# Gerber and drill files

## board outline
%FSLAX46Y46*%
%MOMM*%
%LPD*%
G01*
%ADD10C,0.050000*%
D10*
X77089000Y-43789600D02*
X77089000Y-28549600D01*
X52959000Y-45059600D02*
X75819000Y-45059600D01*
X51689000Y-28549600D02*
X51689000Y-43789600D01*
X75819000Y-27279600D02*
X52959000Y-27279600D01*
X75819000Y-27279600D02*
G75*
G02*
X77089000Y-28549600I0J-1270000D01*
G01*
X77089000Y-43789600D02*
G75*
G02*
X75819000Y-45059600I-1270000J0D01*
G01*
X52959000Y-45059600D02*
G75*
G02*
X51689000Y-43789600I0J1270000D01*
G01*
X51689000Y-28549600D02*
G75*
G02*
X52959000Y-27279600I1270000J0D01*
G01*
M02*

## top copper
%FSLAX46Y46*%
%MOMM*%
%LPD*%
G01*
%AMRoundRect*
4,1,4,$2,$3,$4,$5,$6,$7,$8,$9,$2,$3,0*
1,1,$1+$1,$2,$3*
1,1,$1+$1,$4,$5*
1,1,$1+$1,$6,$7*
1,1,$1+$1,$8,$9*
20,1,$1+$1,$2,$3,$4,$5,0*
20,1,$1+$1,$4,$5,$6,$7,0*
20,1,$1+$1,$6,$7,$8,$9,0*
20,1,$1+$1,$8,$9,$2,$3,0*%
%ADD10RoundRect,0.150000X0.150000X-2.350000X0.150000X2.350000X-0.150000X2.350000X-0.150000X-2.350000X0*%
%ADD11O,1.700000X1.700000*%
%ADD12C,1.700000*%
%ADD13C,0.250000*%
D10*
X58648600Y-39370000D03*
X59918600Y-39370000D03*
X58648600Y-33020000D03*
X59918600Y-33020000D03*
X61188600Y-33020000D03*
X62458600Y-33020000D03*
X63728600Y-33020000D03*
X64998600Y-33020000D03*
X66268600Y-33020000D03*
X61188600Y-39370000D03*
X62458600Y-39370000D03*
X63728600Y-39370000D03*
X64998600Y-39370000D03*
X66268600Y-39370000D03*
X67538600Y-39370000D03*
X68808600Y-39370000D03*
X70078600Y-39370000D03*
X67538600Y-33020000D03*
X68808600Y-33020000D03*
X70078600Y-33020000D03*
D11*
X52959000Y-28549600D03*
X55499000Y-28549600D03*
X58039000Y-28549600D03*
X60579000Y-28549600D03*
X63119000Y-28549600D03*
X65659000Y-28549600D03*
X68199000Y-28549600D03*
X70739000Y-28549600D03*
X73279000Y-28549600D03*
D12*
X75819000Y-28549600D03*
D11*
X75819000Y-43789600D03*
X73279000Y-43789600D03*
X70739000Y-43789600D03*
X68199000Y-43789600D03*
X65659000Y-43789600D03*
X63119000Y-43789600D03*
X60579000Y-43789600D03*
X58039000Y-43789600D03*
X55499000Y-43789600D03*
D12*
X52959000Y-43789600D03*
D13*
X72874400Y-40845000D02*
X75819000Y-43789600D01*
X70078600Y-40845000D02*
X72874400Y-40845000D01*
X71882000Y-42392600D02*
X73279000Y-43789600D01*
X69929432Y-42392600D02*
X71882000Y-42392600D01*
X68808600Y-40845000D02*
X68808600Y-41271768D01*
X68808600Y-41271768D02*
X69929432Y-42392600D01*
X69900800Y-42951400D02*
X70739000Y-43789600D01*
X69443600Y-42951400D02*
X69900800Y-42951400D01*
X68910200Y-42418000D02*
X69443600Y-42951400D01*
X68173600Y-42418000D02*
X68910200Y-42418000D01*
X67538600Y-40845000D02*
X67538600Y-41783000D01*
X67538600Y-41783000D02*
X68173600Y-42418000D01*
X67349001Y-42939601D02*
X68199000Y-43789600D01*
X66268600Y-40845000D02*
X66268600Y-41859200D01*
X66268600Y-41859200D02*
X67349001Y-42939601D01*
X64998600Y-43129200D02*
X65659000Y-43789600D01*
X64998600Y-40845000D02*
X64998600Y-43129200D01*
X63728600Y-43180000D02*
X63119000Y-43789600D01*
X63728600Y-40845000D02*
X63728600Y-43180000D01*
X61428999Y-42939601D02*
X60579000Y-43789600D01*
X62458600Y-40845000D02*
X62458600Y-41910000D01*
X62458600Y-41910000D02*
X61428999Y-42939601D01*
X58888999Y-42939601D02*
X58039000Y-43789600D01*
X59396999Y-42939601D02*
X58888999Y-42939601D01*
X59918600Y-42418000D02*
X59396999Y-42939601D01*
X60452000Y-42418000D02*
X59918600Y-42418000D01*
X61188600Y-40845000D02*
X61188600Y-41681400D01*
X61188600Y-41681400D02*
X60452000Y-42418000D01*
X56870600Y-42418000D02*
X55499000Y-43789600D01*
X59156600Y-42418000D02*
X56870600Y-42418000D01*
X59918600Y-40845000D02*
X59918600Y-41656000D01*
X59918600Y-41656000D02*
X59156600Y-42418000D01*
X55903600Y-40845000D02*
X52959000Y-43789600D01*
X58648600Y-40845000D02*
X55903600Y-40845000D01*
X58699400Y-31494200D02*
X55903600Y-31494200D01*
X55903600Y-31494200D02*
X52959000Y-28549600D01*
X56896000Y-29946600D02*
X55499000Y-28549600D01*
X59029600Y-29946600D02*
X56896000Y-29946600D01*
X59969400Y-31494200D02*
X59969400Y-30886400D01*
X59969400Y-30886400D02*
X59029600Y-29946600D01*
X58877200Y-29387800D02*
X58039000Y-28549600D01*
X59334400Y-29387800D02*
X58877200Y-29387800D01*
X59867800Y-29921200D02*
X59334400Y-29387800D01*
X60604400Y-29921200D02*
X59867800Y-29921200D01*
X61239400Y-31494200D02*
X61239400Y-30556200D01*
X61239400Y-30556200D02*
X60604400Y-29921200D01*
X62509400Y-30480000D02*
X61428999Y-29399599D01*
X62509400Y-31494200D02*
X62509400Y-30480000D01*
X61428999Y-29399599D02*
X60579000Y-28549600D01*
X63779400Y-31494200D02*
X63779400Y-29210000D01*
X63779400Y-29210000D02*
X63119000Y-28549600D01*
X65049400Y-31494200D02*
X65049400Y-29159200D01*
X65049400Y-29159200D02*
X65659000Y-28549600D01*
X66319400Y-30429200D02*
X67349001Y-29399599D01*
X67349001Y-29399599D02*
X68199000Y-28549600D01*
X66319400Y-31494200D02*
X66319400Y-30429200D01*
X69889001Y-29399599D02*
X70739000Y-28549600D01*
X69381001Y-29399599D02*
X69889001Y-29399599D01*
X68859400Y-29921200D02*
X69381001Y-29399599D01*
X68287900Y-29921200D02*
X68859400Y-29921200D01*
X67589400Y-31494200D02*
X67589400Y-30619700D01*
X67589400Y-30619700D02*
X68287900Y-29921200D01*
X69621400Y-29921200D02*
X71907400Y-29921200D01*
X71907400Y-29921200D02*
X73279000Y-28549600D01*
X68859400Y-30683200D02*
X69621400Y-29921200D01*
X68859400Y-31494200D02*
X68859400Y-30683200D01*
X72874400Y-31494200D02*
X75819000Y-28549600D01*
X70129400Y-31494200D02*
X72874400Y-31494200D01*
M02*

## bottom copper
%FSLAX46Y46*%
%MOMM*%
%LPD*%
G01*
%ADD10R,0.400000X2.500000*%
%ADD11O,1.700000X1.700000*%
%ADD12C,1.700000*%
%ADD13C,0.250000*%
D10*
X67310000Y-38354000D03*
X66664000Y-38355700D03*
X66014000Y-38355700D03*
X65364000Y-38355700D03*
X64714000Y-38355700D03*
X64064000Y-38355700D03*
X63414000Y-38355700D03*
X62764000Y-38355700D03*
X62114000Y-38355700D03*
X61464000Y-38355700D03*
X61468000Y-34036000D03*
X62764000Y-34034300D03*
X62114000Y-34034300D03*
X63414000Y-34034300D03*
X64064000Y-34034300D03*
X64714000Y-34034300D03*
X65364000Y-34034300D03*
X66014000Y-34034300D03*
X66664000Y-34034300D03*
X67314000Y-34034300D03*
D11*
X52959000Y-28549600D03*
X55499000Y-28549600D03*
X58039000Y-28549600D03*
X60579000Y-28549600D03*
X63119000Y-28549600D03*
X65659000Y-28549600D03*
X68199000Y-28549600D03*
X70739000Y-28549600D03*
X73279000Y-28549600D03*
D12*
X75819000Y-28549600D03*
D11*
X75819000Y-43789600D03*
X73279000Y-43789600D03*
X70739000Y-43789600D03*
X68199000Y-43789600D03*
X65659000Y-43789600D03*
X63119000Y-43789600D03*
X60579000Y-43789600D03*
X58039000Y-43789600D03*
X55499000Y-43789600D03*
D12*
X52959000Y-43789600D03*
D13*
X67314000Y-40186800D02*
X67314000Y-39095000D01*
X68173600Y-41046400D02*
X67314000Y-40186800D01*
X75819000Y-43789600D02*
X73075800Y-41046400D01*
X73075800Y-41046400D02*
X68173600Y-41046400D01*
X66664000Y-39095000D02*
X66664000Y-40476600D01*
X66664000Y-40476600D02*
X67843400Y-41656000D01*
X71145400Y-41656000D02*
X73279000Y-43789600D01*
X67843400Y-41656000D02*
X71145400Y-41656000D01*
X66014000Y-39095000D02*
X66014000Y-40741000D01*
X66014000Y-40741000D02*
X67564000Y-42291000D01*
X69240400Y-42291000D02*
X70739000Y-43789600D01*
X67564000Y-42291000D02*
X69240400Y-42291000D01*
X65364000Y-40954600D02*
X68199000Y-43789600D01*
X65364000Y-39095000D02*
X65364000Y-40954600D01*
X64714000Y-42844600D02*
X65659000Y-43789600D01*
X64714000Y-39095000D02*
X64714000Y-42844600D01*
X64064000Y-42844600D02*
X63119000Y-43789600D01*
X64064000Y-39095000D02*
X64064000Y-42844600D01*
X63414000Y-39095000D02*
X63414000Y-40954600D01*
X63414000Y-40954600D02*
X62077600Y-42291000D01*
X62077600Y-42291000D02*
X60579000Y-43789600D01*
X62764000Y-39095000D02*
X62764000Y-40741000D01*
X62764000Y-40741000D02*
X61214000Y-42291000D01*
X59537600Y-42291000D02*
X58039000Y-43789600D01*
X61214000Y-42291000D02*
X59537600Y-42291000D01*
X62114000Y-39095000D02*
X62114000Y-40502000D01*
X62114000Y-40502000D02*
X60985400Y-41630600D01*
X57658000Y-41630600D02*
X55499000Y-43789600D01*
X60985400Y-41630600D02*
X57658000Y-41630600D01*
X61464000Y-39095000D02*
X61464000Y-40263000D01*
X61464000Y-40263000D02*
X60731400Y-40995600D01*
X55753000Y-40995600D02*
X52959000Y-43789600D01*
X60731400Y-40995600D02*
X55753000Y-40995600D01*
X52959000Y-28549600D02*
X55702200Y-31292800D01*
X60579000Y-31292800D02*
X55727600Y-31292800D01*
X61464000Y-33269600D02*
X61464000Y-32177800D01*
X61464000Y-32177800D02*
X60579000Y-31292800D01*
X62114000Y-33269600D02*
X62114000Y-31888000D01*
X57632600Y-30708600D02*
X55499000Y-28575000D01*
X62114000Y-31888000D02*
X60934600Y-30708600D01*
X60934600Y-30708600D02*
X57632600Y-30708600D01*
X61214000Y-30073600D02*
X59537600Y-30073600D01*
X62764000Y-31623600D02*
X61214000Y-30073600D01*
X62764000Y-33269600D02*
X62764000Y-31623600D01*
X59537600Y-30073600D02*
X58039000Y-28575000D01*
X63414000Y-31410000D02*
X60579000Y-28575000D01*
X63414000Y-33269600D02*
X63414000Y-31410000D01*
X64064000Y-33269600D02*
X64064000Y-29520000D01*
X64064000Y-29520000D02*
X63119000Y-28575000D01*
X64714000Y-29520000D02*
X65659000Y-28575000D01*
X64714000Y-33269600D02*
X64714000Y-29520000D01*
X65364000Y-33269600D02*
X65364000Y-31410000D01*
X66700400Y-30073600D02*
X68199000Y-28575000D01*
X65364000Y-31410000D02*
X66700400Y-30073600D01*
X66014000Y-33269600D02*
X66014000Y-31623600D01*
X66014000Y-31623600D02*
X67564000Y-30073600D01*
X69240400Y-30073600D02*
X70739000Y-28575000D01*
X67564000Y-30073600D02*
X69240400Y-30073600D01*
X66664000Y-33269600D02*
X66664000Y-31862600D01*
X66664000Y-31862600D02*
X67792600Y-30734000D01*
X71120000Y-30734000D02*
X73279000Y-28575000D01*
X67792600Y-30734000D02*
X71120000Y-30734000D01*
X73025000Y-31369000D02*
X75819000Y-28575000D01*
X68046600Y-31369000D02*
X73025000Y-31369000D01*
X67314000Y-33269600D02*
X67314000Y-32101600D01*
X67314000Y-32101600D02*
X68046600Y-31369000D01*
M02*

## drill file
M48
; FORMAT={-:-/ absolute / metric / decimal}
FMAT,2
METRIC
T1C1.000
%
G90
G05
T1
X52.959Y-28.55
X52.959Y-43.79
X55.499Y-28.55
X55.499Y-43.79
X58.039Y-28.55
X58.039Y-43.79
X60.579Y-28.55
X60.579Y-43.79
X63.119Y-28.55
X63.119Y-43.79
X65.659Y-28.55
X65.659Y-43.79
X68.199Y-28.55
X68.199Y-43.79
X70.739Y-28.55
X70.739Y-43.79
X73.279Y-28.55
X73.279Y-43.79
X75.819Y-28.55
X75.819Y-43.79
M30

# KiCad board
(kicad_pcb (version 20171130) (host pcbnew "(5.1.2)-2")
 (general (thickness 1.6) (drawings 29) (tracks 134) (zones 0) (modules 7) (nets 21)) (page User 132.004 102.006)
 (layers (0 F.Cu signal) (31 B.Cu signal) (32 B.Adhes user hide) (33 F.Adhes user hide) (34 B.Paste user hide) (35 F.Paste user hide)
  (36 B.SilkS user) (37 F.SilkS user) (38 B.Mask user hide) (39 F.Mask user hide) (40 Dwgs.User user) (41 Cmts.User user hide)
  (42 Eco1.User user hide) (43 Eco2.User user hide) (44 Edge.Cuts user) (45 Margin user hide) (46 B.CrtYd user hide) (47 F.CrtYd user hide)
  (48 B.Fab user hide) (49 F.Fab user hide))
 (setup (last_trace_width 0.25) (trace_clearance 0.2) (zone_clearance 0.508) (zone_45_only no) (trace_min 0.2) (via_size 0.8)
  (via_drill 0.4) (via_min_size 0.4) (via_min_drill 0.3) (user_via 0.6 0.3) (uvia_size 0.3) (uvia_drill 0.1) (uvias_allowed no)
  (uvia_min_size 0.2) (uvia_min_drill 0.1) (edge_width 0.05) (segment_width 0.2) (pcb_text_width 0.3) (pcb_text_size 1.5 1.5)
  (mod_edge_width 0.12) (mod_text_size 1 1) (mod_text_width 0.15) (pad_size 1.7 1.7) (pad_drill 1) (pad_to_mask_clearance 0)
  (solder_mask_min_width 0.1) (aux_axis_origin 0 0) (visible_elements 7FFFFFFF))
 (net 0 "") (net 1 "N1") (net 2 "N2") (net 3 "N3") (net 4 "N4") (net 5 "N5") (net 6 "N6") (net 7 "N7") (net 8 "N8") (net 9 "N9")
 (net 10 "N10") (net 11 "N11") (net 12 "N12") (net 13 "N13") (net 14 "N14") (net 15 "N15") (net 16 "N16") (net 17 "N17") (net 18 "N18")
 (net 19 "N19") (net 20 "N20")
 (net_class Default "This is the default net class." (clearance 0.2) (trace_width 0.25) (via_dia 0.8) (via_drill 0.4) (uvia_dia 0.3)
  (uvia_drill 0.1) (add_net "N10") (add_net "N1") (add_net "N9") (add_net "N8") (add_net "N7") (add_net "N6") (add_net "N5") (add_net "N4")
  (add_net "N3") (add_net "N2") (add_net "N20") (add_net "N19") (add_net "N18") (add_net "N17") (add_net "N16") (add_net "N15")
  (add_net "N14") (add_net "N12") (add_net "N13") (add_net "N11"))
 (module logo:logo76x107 (layer B.Cu) (at 72.4535 36.322 90)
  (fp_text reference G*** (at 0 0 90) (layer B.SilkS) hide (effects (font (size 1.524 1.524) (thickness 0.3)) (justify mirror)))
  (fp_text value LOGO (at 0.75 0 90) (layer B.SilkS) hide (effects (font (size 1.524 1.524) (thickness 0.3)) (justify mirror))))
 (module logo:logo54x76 (layer F.Cu) (at 54.864 36.195 90)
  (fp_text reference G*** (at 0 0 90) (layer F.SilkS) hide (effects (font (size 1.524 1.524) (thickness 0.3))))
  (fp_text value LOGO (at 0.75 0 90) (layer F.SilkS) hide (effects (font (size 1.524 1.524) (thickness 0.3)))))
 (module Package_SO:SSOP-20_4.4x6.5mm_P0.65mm (layer B.Cu) (at 64.389 36.195 90)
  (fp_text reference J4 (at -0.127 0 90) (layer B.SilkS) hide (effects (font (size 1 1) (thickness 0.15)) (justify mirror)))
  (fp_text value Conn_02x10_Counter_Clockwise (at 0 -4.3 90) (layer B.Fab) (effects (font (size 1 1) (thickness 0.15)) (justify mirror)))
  (pad 1 smd rect (at -2.159 2.921 90) (size 2.5 0.4) (layers B.Cu B.Paste B.Mask) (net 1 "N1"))
  (pad 2 smd rect (at -2.1607 2.275 90) (size 2.5 0.4) (layers B.Cu B.Paste B.Mask) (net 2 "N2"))
  (pad 3 smd rect (at -2.1607 1.625 90) (size 2.5 0.4) (layers B.Cu B.Paste B.Mask) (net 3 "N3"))
  (pad 4 smd rect (at -2.1607 0.975 90) (size 2.5 0.4) (layers B.Cu B.Paste B.Mask) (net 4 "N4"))
  (pad 5 smd rect (at -2.1607 0.325 90) (size 2.5 0.4) (layers B.Cu B.Paste B.Mask) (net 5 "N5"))
  (pad 6 smd rect (at -2.1607 -0.325 90) (size 2.5 0.4) (layers B.Cu B.Paste B.Mask) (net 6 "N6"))
  (pad 7 smd rect (at -2.1607 -0.975 90) (size 2.5 0.4) (layers B.Cu B.Paste B.Mask) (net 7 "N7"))
  (pad 8 smd rect (at -2.1607 -1.625 90) (size 2.5 0.4) (layers B.Cu B.Paste B.Mask) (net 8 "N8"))
  (pad 9 smd rect (at -2.1607 -2.275 90) (size 2.5 0.4) (layers B.Cu B.Paste B.Mask) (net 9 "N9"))
  (pad 10 smd rect (at -2.1607 -2.925 90) (size 2.5 0.4) (layers B.Cu B.Paste B.Mask) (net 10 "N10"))
  (pad 11 smd rect (at 2.159 -2.921 270) (size 2.5 0.4) (layers B.Cu B.Paste B.Mask) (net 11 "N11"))
  (pad 13 smd rect (at 2.1607 -1.625 270) (size 2.5 0.4) (layers B.Cu B.Paste B.Mask) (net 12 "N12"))
  (pad 12 smd rect (at 2.1607 -2.275 270) (size 2.5 0.4) (layers B.Cu B.Paste B.Mask) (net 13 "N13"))
  (pad 14 smd rect (at 2.1607 -0.975 270) (size 2.5 0.4) (layers B.Cu B.Paste B.Mask) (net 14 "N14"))
  (pad 15 smd rect (at 2.1607 -0.325 270) (size 2.5 0.4) (layers B.Cu B.Paste B.Mask) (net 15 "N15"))
  (pad 16 smd rect (at 2.1607 0.325 270) (size 2.5 0.4) (layers B.Cu B.Paste B.Mask) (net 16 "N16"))
  (pad 17 smd rect (at 2.1607 0.975 270) (size 2.5 0.4) (layers B.Cu B.Paste B.Mask) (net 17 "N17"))
  (pad 18 smd rect (at 2.1607 1.625 270) (size 2.5 0.4) (layers B.Cu B.Paste B.Mask) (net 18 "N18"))
  (pad 19 smd rect (at 2.1607 2.275 270) (size 2.5 0.4) (layers B.Cu B.Paste B.Mask) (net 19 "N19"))
  (pad 20 smd rect (at 2.1607 2.925 270) (size 2.5 0.4) (layers B.Cu B.Paste B.Mask) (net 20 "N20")))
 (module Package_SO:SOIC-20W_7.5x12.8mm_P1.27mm (layer F.Cu) (at 64.3636 36.195 90)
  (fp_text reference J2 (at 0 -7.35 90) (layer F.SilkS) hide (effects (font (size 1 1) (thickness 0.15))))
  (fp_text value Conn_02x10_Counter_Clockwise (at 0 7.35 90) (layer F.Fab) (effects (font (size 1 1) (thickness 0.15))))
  (pad 1 smd roundrect (at -3.175 -5.715 90) (size 5 0.6) (layers F.Cu F.Paste F.Mask) (roundrect_rratio 0.25) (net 10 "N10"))
  (pad 2 smd roundrect (at -3.175 -4.445 90) (size 5 0.6) (layers F.Cu F.Paste F.Mask) (roundrect_rratio 0.25) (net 9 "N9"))
  (pad 20 smd roundrect (at 3.175 -5.715 90) (size 5 0.6) (layers F.Cu F.Paste F.Mask) (roundrect_rratio 0.25) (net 11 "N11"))
  (pad 19 smd roundrect (at 3.175 -4.445 90) (size 5 0.6) (layers F.Cu F.Paste F.Mask) (roundrect_rratio 0.25) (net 13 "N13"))
  (pad 18 smd roundrect (at 3.175 -3.175 90) (size 5 0.6) (layers F.Cu F.Paste F.Mask) (roundrect_rratio 0.25) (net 12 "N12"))
  (pad 17 smd roundrect (at 3.175 -1.905 90) (size 5 0.6) (layers F.Cu F.Paste F.Mask) (roundrect_rratio 0.25) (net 14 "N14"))
  (pad 16 smd roundrect (at 3.175 -0.635 90) (size 5 0.6) (layers F.Cu F.Paste F.Mask) (roundrect_rratio 0.25) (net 15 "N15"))
  (pad 15 smd roundrect (at 3.175 0.635 90) (size 5 0.6) (layers F.Cu F.Paste F.Mask) (roundrect_rratio 0.25) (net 16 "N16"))
  (pad 14 smd roundrect (at 3.175 1.905 90) (size 5 0.6) (layers F.Cu F.Paste F.Mask) (roundrect_rratio 0.25) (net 17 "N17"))
  (pad 3 smd roundrect (at -3.175 -3.175 90) (size 5 0.6) (layers F.Cu F.Paste F.Mask) (roundrect_rratio 0.25) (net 8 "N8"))
  (pad 4 smd roundrect (at -3.175 -1.905 90) (size 5 0.6) (layers F.Cu F.Paste F.Mask) (roundrect_rratio 0.25) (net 7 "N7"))
  (pad 5 smd roundrect (at -3.175 -0.635 90) (size 5 0.6) (layers F.Cu F.Paste F.Mask) (roundrect_rratio 0.25) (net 6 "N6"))
  (pad 6 smd roundrect (at -3.175 0.635 90) (size 5 0.6) (layers F.Cu F.Paste F.Mask) (roundrect_rratio 0.25) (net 5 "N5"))
  (pad 7 smd roundrect (at -3.175 1.905 90) (size 5 0.6) (layers F.Cu F.Paste F.Mask) (roundrect_rratio 0.25) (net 4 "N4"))
  (pad 8 smd roundrect (at -3.175 3.175 90) (size 5 0.6) (layers F.Cu F.Paste F.Mask) (roundrect_rratio 0.25) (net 3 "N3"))
  (pad 9 smd roundrect (at -3.175 4.445 90) (size 5 0.6) (layers F.Cu F.Paste F.Mask) (roundrect_rratio 0.25) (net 2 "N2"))
  (pad 10 smd roundrect (at -3.175 5.715 90) (size 5 0.6) (layers F.Cu F.Paste F.Mask) (roundrect_rratio 0.25) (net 1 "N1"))
  (pad 13 smd roundrect (at 3.175 3.175 90) (size 5 0.6) (layers F.Cu F.Paste F.Mask) (roundrect_rratio 0.25) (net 18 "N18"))
  (pad 12 smd roundrect (at 3.175 4.445 90) (size 5 0.6) (layers F.Cu F.Paste F.Mask) (roundrect_rratio 0.25) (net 19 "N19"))
  (pad 11 smd roundrect (at 3.175 5.715 90) (size 5 0.6) (layers F.Cu F.Paste F.Mask) (roundrect_rratio 0.25) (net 20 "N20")))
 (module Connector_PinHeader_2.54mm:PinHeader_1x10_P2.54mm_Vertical (layer B.Cu) (at 75.819 28.5496 90)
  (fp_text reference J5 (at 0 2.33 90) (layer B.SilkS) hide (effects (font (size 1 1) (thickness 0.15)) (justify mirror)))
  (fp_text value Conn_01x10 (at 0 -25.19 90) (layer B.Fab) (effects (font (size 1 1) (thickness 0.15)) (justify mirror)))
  (pad 10 thru_hole oval (at 0 -22.86 90) (size 1.7 1.7) (drill 1) (layers *.Cu *.Mask) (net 11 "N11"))
  (pad 9 thru_hole oval (at 0 -20.32 90) (size 1.7 1.7) (drill 1) (layers *.Cu *.Mask) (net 13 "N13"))
  (pad 8 thru_hole oval (at 0 -17.78 90) (size 1.7 1.7) (drill 1) (layers *.Cu *.Mask) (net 12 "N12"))
  (pad 7 thru_hole oval (at 0 -15.24 90) (size 1.7 1.7) (drill 1) (layers *.Cu *.Mask) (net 14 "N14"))
  (pad 6 thru_hole oval (at 0 -12.7 90) (size 1.7 1.7) (drill 1) (layers *.Cu *.Mask) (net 15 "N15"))
  (pad 5 thru_hole oval (at 0 -10.16 90) (size 1.7 1.7) (drill 1) (layers *.Cu *.Mask) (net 16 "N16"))
  (pad 4 thru_hole oval (at 0 -7.62 90) (size 1.7 1.7) (drill 1) (layers *.Cu *.Mask) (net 17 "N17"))
  (pad 3 thru_hole oval (at 0 -5.08 90) (size 1.7 1.7) (drill 1) (layers *.Cu *.Mask) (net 18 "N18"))
  (pad 2 thru_hole oval (at 0 -2.54 90) (size 1.7 1.7) (drill 1) (layers *.Cu *.Mask) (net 19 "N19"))
  (pad 1 thru_hole circle (at 0 0 90) (size 1.7 1.7) (drill 1) (layers *.Cu *.Mask) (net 20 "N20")))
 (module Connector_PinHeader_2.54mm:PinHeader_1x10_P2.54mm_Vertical (layer B.Cu) (at 52.959 43.7896 270)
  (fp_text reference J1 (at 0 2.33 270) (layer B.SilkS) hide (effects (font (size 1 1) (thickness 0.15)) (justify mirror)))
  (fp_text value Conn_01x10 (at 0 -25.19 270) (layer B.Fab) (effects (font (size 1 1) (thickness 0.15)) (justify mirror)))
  (pad 10 thru_hole oval (at 0 -22.86 270) (size 1.7 1.7) (drill 1) (layers *.Cu *.Mask) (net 1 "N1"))
  (pad 9 thru_hole oval (at 0 -20.32 270) (size 1.7 1.7) (drill 1) (layers *.Cu *.Mask) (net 2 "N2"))
  (pad 8 thru_hole oval (at 0 -17.78 270) (size 1.7 1.7) (drill 1) (layers *.Cu *.Mask) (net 3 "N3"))
  (pad 7 thru_hole oval (at 0 -15.24 270) (size 1.7 1.7) (drill 1) (layers *.Cu *.Mask) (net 4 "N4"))
  (pad 6 thru_hole oval (at 0 -12.7 270) (size 1.7 1.7) (drill 1) (layers *.Cu *.Mask) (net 5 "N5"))
  (pad 5 thru_hole oval (at 0 -10.16 270) (size 1.7 1.7) (drill 1) (layers *.Cu *.Mask) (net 6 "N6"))
  (pad 4 thru_hole oval (at 0 -7.62 270) (size 1.7 1.7) (drill 1) (layers *.Cu *.Mask) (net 7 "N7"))
  (pad 3 thru_hole oval (at 0 -5.08 270) (size 1.7 1.7) (drill 1) (layers *.Cu *.Mask) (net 8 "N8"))
  (pad 2 thru_hole oval (at 0 -2.54 270) (size 1.7 1.7) (drill 1) (layers *.Cu *.Mask) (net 9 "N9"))
  (pad 1 thru_hole circle (at 0 0 270) (size 1.7 1.7) (drill 1) (layers *.Cu *.Mask) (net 10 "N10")))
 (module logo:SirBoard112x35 (layer B.Cu) (at 57.1246 36.195 90)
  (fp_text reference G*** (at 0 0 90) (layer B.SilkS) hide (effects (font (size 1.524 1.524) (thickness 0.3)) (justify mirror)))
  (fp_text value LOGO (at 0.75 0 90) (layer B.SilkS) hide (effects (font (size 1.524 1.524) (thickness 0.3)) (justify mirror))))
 (gr_line (start 77.089 43.7896) (end 77.089 28.5496) (layer Edge.Cuts) (width 0.05))
 (gr_line (start 52.959 45.0596) (end 75.819 45.0596) (layer Edge.Cuts) (width 0.05))
 (gr_line (start 51.689 28.5496) (end 51.689 43.7896) (layer Edge.Cuts) (width 0.05))
 (gr_line (start 75.819 27.2796) (end 52.959 27.2796) (layer Edge.Cuts) (width 0.05))
 (gr_arc (start 75.819 28.5496) (end 77.089 28.5496) (angle -90) (layer Edge.Cuts) (width 0.05))
 (gr_arc (start 75.819 43.7896) (end 75.819 45.0596) (angle -90) (layer Edge.Cuts) (width 0.05))
 (gr_arc (start 52.959 43.7896) (end 51.689 43.7896) (angle -90) (layer Edge.Cuts) (width 0.05))
 (gr_arc (start 52.959 28.5496) (end 52.959 27.2796) (angle -90) (layer Edge.Cuts) (width 0.05))
 (segment (start 72.8744 40.845) (end 75.819 43.7896) (width 0.25) (layer F.Cu) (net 1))
 (segment (start 70.0786 40.845) (end 72.8744 40.845) (width 0.25) (layer F.Cu) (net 1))
 (segment (start 67.314 40.1868) (end 67.314 39.095) (width 0.25) (layer B.Cu) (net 1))
 (segment (start 68.1736 41.0464) (end 67.314 40.1868) (width 0.25) (layer B.Cu) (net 1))
 (segment (start 75.819 43.7896) (end 73.0758 41.0464) (width 0.25) (layer B.Cu) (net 1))
 (segment (start 73.0758 41.0464) (end 68.1736 41.0464) (width 0.25) (layer B.Cu) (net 1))
 (segment (start 66.664 39.095) (end 66.664 40.4766) (width 0.25) (layer B.Cu) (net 2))
 (segment (start 66.664 40.4766) (end 67.8434 41.656) (width 0.25) (layer B.Cu) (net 2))
 (segment (start 71.1454 41.656) (end 73.279 43.7896) (width 0.25) (layer B.Cu) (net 2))
 (segment (start 67.8434 41.656) (end 71.1454 41.656) (width 0.25) (layer B.Cu) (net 2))
 (segment (start 71.882 42.3926) (end 73.279 43.7896) (width 0.25) (layer F.Cu) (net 2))
 (segment (start 69.929432 42.3926) (end 71.882 42.3926) (width 0.25) (layer F.Cu) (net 2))
 (segment (start 68.8086 40.845) (end 68.8086 41.271768) (width 0.25) (layer F.Cu) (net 2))
 (segment (start 68.8086 41.271768) (end 69.929432 42.3926) (width 0.25) (layer F.Cu) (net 2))
 (segment (start 66.014 39.095) (end 66.014 40.741) (width 0.25) (layer B.Cu) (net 3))
 (segment (start 66.014 40.741) (end 67.564 42.291) (width 0.25) (layer B.Cu) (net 3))
 (segment (start 69.2404 42.291) (end 70.739 43.7896) (width 0.25) (layer B.Cu) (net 3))
 (segment (start 67.564 42.291) (end 69.2404 42.291) (width 0.25) (layer B.Cu) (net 3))
 (segment (start 69.9008 42.9514) (end 70.739 43.7896) (width 0.25) (layer F.Cu) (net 3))
 (segment (start 69.4436 42.9514) (end 69.9008 42.9514) (width 0.25) (layer F.Cu) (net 3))
 (segment (start 68.9102 42.418) (end 69.4436 42.9514) (width 0.25) (layer F.Cu) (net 3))
 (segment (start 68.1736 42.418) (end 68.9102 42.418) (width 0.25) (layer F.Cu) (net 3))
 (segment (start 67.5386 40.845) (end 67.5386 41.783) (width 0.25) (layer F.Cu) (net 3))
 (segment (start 67.5386 41.783) (end 68.1736 42.418) (width 0.25) (layer F.Cu) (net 3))
 (segment (start 65.364 40.9546) (end 68.199 43.7896) (width 0.25) (layer B.Cu) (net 4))
 (segment (start 65.364 39.095) (end 65.364 40.9546) (width 0.25) (layer B.Cu) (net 4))
 (segment (start 67.349001 42.939601) (end 68.199 43.7896) (width 0.25) (layer F.Cu) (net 4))
 (segment (start 66.2686 40.845) (end 66.2686 41.8592) (width 0.25) (layer F.Cu) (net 4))
 (segment (start 66.2686 41.8592) (end 67.349001 42.939601) (width 0.25) (layer F.Cu) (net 4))
 (segment (start 64.714 42.8446) (end 65.659 43.7896) (width 0.25) (layer B.Cu) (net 5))
 (segment (start 64.714 39.095) (end 64.714 42.8446) (width 0.25) (layer B.Cu) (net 5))
 (segment (start 64.9986 43.1292) (end 65.659 43.7896) (width 0.25) (layer F.Cu) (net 5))
 (segment (start 64.9986 40.845) (end 64.9986 43.1292) (width 0.25) (layer F.Cu) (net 5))
 (segment (start 64.064 42.8446) (end 63.119 43.7896) (width 0.25) (layer B.Cu) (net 6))
 (segment (start 64.064 39.095) (end 64.064 42.8446) (width 0.25) (layer B.Cu) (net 6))
 (segment (start 63.7286 43.18) (end 63.119 43.7896) (width 0.25) (layer F.Cu) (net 6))
 (segment (start 63.7286 40.845) (end 63.7286 43.18) (width 0.25) (layer F.Cu) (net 6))
 (segment (start 63.414 39.095) (end 63.414 40.9546) (width 0.25) (layer B.Cu) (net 7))
 (segment (start 63.414 40.9546) (end 62.0776 42.291) (width 0.25) (layer B.Cu) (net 7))
 (segment (start 62.0776 42.291) (end 60.579 43.7896) (width 0.25) (layer B.Cu) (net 7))
 (segment (start 61.428999 42.939601) (end 60.579 43.7896) (width 0.25) (layer F.Cu) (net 7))
 (segment (start 62.4586 40.845) (end 62.4586 41.91) (width 0.25) (layer F.Cu) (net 7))
 (segment (start 62.4586 41.91) (end 61.428999 42.939601) (width 0.25) (layer F.Cu) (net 7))
 (segment (start 62.764 39.095) (end 62.764 40.741) (width 0.25) (layer B.Cu) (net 8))
 (segment (start 62.764 40.741) (end 61.214 42.291) (width 0.25) (layer B.Cu) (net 8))
 (segment (start 59.5376 42.291) (end 58.039 43.7896) (width 0.25) (layer B.Cu) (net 8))
 (segment (start 61.214 42.291) (end 59.5376 42.291) (width 0.25) (layer B.Cu) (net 8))
 (segment (start 58.888999 42.939601) (end 58.039 43.7896) (width 0.25) (layer F.Cu) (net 8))
 (segment (start 59.396999 42.939601) (end 58.888999 42.939601) (width 0.25) (layer F.Cu) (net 8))
 (segment (start 59.9186 42.418) (end 59.396999 42.939601) (width 0.25) (layer F.Cu) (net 8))
 (segment (start 60.452 42.418) (end 59.9186 42.418) (width 0.25) (layer F.Cu) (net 8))
 (segment (start 61.1886 40.845) (end 61.1886 41.6814) (width 0.25) (layer F.Cu) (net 8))
 (segment (start 61.1886 41.6814) (end 60.452 42.418) (width 0.25) (layer F.Cu) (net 8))
 (segment (start 62.114 39.095) (end 62.114 40.502) (width 0.25) (layer B.Cu) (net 9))
 (segment (start 62.114 40.502) (end 60.9854 41.6306) (width 0.25) (layer B.Cu) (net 9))
 (segment (start 57.658 41.6306) (end 55.499 43.7896) (width 0.25) (layer B.Cu) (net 9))
 (segment (start 60.9854 41.6306) (end 57.658 41.6306) (width 0.25) (layer B.Cu) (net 9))
 (segment (start 56.8706 42.418) (end 55.499 43.7896) (width 0.25) (layer F.Cu) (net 9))
 (segment (start 59.1566 42.418) (end 56.8706 42.418) (width 0.25) (layer F.Cu) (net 9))
 (segment (start 59.9186 40.845) (end 59.9186 41.656) (width 0.25) (layer F.Cu) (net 9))
 (segment (start 59.9186 41.656) (end 59.1566 42.418) (width 0.25) (layer F.Cu) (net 9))
 (segment (start 61.464 39.095) (end 61.464 40.263) (width 0.25) (layer B.Cu) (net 10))
 (segment (start 61.464 40.263) (end 60.7314 40.9956) (width 0.25) (layer B.Cu) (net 10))
 (segment (start 55.753 40.9956) (end 52.959 43.7896) (width 0.25) (layer B.Cu) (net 10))
 (segment (start 60.7314 40.9956) (end 55.753 40.9956) (width 0.25) (layer B.Cu) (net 10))
 (segment (start 55.9036 40.845) (end 52.959 43.7896) (width 0.25) (layer F.Cu) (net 10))
 (segment (start 58.6486 40.845) (end 55.9036 40.845) (width 0.25) (layer F.Cu) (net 10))
 (segment (start 52.959 28.5496) (end 55.7022 31.2928) (width 0.25) (layer B.Cu) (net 11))
 (segment (start 58.6994 31.4942) (end 55.9036 31.4942) (width 0.25) (layer F.Cu) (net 11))
 (segment (start 55.9036 31.4942) (end 52.959 28.5496) (width 0.25) (layer F.Cu) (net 11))
 (segment (start 60.579 31.2928) (end 55.7276 31.2928) (width 0.25) (layer B.Cu) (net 11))
 (segment (start 61.464 33.2696) (end 61.464 32.1778) (width 0.25) (layer B.Cu) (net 11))
 (segment (start 61.464 32.1778) (end 60.579 31.2928) (width 0.25) (layer B.Cu) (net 11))
 (segment (start 62.114 33.2696) (end 62.114 31.888) (width 0.25) (layer B.Cu) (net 13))
 (segment (start 57.6326 30.7086) (end 55.499 28.575) (width 0.25) (layer B.Cu) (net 13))
 (segment (start 62.114 31.888) (end 60.9346 30.7086) (width 0.25) (layer B.Cu) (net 13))
 (segment (start 60.9346 30.7086) (end 57.6326 30.7086) (width 0.25) (layer B.Cu) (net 13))
 (segment (start 56.896 29.9466) (end 55.499 28.5496) (width 0.25) (layer F.Cu) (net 13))
 (segment (start 59.0296 29.9466) (end 56.896 29.9466) (width 0.25) (layer F.Cu) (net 13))
 (segment (start 59.9694 31.4942) (end 59.9694 30.8864) (width 0.25) (layer F.Cu) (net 13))
 (segment (start 59.9694 30.8864) (end 59.0296 29.9466) (width 0.25) (layer F.Cu) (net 13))
 (segment (start 61.214 30.0736) (end 59.5376 30.0736) (width 0.25) (layer B.Cu) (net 12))
 (segment (start 62.764 31.6236) (end 61.214 30.0736) (width 0.25) (layer B.Cu) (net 12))
 (segment (start 62.764 33.2696) (end 62.764 31.6236) (width 0.25) (layer B.Cu) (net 12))
 (segment (start 59.5376 30.0736) (end 58.039 28.575) (width 0.25) (layer B.Cu) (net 12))
 (segment (start 58.8772 29.3878) (end 58.039 28.5496) (width 0.25) (layer F.Cu) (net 12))
 (segment (start 59.3344 29.3878) (end 58.8772 29.3878) (width 0.25) (layer F.Cu) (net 12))
 (segment (start 59.8678 29.9212) (end 59.3344 29.3878) (width 0.25) (layer F.Cu) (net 12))
 (segment (start 60.6044 29.9212) (end 59.8678 29.9212) (width 0.25) (layer F.Cu) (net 12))
 (segment (start 61.2394 31.4942) (end 61.2394 30.5562) (width 0.25) (layer F.Cu) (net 12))
 (segment (start 61.2394 30.5562) (end 60.6044 29.9212) (width 0.25) (layer F.Cu) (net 12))
 (segment (start 62.5094 30.48) (end 61.428999 29.399599) (width 0.25) (layer F.Cu) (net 14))
 (segment (start 62.5094 31.4942) (end 62.5094 30.48) (width 0.25) (layer F.Cu) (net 14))
 (segment (start 61.428999 29.399599) (end 60.579 28.5496) (width 0.25) (layer F.Cu) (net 14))
 (segment (start 63.414 31.41) (end 60.579 28.575) (width 0.25) (layer B.Cu) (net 14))
 (segment (start 63.414 33.2696) (end 63.414 31.41) (width 0.25) (layer B.Cu) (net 14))
 (segment (start 63.7794 31.4942) (end 63.7794 29.21) (width 0.25) (layer F.Cu) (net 15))
 (segment (start 63.7794 29.21) (end 63.119 28.5496) (width 0.25) (layer F.Cu) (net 15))
 (segment (start 64.064 33.2696) (end 64.064 29.52) (width 0.25) (layer B.Cu) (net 15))
 (segment (start 64.064 29.52) (end 63.119 28.575) (width 0.25) (layer B.Cu) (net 15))
 (segment (start 65.0494 31.4942) (end 65.0494 29.1592) (width 0.25) (layer F.Cu) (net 16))
 (segment (start 65.0494 29.1592) (end 65.659 28.5496) (width 0.25) (layer F.Cu) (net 16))
 (segment (start 64.714 29.52) (end 65.659 28.575) (width 0.25) (layer B.Cu) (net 16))
 (segment (start 64.714 33.2696) (end 64.714 29.52) (width 0.25) (layer B.Cu) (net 16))
 (segment (start 66.3194 30.4292) (end 67.349001 29.399599) (width 0.25) (layer F.Cu) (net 17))
 (segment (start 67.349001 29.399599) (end 68.199 28.5496) (width 0.25) (layer F.Cu) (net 17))
 (segment (start 66.3194 31.4942) (end 66.3194 30.4292) (width 0.25) (layer F.Cu) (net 17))
 (segment (start 65.364 33.2696) (end 65.364 31.41) (width 0.25) (layer B.Cu) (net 17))
 (segment (start 66.7004 30.0736) (end 68.199 28.575) (width 0.25) (layer B.Cu) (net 17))
 (segment (start 65.364 31.41) (end 66.7004 30.0736) (width 0.25) (layer B.Cu) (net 17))
 (segment (start 66.014 33.2696) (end 66.014 31.6236) (width 0.25) (layer B.Cu) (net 18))
 (segment (start 66.014 31.6236) (end 67.564 30.0736) (width 0.25) (layer B.Cu) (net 18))
 (segment (start 69.2404 30.0736) (end 70.739 28.575) (width 0.25) (layer B.Cu) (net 18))
 (segment (start 67.564 30.0736) (end 69.2404 30.0736) (width 0.25) (layer B.Cu) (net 18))
 (segment (start 69.889001 29.399599) (end 70.739 28.5496) (width 0.25) (layer F.Cu) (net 18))
 (segment (start 69.381001 29.399599) (end 69.889001 29.399599) (width 0.25) (layer F.Cu) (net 18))
 (segment (start 68.8594 29.9212) (end 69.381001 29.399599) (width 0.25) (layer F.Cu) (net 18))
 (segment (start 68.2879 29.9212) (end 68.8594 29.9212) (width 0.25) (layer F.Cu) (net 18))
 (segment (start 67.5894 31.4942) (end 67.5894 30.6197) (width 0.25) (layer F.Cu) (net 18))
 (segment (start 67.5894 30.6197) (end 68.2879 29.9212) (width 0.25) (layer F.Cu) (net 18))
 (segment (start 69.6214 29.9212) (end 71.9074 29.9212) (width 0.25) (layer F.Cu) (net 19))
 (segment (start 71.9074 29.9212) (end 73.279 28.5496) (width 0.25) (layer F.Cu) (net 19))
 (segment (start 68.8594 30.6832) (end 69.6214 29.9212) (width 0.25) (layer F.Cu) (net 19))
 (segment (start 68.8594 31.4942) (end 68.8594 30.6832) (width 0.25) (layer F.Cu) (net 19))
 (segment (start 66.664 33.2696) (end 66.664 31.8626) (width 0.25) (layer B.Cu) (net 19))
 (segment (start 66.664 31.8626) (end 67.7926 30.734) (width 0.25) (layer B.Cu) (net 19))
 (segment (start 71.12 30.734) (end 73.279 28.575) (width 0.25) (layer B.Cu) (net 19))
 (segment (start 67.7926 30.734) (end 71.12 30.734) (width 0.25) (layer B.Cu) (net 19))
 (segment (start 72.8744 31.4942) (end 75.819 28.5496) (width 0.25) (layer F.Cu) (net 20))
 (segment (start 70.1294 31.4942) (end 72.8744 31.4942) (width 0.25) (layer F.Cu) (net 20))
 (segment (start 73.025 31.369) (end 75.819 28.575) (width 0.25) (layer B.Cu) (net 20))
 (segment (start 68.0466 31.369) (end 73.025 31.369) (width 0.25) (layer B.Cu) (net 20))
 (segment (start 67.314 33.2696) (end 67.314 32.1016) (width 0.25) (layer B.Cu) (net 20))
 (segment (start 67.314 32.1016) (end 68.0466 31.369) (width 0.25) (layer B.Cu) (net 20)))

